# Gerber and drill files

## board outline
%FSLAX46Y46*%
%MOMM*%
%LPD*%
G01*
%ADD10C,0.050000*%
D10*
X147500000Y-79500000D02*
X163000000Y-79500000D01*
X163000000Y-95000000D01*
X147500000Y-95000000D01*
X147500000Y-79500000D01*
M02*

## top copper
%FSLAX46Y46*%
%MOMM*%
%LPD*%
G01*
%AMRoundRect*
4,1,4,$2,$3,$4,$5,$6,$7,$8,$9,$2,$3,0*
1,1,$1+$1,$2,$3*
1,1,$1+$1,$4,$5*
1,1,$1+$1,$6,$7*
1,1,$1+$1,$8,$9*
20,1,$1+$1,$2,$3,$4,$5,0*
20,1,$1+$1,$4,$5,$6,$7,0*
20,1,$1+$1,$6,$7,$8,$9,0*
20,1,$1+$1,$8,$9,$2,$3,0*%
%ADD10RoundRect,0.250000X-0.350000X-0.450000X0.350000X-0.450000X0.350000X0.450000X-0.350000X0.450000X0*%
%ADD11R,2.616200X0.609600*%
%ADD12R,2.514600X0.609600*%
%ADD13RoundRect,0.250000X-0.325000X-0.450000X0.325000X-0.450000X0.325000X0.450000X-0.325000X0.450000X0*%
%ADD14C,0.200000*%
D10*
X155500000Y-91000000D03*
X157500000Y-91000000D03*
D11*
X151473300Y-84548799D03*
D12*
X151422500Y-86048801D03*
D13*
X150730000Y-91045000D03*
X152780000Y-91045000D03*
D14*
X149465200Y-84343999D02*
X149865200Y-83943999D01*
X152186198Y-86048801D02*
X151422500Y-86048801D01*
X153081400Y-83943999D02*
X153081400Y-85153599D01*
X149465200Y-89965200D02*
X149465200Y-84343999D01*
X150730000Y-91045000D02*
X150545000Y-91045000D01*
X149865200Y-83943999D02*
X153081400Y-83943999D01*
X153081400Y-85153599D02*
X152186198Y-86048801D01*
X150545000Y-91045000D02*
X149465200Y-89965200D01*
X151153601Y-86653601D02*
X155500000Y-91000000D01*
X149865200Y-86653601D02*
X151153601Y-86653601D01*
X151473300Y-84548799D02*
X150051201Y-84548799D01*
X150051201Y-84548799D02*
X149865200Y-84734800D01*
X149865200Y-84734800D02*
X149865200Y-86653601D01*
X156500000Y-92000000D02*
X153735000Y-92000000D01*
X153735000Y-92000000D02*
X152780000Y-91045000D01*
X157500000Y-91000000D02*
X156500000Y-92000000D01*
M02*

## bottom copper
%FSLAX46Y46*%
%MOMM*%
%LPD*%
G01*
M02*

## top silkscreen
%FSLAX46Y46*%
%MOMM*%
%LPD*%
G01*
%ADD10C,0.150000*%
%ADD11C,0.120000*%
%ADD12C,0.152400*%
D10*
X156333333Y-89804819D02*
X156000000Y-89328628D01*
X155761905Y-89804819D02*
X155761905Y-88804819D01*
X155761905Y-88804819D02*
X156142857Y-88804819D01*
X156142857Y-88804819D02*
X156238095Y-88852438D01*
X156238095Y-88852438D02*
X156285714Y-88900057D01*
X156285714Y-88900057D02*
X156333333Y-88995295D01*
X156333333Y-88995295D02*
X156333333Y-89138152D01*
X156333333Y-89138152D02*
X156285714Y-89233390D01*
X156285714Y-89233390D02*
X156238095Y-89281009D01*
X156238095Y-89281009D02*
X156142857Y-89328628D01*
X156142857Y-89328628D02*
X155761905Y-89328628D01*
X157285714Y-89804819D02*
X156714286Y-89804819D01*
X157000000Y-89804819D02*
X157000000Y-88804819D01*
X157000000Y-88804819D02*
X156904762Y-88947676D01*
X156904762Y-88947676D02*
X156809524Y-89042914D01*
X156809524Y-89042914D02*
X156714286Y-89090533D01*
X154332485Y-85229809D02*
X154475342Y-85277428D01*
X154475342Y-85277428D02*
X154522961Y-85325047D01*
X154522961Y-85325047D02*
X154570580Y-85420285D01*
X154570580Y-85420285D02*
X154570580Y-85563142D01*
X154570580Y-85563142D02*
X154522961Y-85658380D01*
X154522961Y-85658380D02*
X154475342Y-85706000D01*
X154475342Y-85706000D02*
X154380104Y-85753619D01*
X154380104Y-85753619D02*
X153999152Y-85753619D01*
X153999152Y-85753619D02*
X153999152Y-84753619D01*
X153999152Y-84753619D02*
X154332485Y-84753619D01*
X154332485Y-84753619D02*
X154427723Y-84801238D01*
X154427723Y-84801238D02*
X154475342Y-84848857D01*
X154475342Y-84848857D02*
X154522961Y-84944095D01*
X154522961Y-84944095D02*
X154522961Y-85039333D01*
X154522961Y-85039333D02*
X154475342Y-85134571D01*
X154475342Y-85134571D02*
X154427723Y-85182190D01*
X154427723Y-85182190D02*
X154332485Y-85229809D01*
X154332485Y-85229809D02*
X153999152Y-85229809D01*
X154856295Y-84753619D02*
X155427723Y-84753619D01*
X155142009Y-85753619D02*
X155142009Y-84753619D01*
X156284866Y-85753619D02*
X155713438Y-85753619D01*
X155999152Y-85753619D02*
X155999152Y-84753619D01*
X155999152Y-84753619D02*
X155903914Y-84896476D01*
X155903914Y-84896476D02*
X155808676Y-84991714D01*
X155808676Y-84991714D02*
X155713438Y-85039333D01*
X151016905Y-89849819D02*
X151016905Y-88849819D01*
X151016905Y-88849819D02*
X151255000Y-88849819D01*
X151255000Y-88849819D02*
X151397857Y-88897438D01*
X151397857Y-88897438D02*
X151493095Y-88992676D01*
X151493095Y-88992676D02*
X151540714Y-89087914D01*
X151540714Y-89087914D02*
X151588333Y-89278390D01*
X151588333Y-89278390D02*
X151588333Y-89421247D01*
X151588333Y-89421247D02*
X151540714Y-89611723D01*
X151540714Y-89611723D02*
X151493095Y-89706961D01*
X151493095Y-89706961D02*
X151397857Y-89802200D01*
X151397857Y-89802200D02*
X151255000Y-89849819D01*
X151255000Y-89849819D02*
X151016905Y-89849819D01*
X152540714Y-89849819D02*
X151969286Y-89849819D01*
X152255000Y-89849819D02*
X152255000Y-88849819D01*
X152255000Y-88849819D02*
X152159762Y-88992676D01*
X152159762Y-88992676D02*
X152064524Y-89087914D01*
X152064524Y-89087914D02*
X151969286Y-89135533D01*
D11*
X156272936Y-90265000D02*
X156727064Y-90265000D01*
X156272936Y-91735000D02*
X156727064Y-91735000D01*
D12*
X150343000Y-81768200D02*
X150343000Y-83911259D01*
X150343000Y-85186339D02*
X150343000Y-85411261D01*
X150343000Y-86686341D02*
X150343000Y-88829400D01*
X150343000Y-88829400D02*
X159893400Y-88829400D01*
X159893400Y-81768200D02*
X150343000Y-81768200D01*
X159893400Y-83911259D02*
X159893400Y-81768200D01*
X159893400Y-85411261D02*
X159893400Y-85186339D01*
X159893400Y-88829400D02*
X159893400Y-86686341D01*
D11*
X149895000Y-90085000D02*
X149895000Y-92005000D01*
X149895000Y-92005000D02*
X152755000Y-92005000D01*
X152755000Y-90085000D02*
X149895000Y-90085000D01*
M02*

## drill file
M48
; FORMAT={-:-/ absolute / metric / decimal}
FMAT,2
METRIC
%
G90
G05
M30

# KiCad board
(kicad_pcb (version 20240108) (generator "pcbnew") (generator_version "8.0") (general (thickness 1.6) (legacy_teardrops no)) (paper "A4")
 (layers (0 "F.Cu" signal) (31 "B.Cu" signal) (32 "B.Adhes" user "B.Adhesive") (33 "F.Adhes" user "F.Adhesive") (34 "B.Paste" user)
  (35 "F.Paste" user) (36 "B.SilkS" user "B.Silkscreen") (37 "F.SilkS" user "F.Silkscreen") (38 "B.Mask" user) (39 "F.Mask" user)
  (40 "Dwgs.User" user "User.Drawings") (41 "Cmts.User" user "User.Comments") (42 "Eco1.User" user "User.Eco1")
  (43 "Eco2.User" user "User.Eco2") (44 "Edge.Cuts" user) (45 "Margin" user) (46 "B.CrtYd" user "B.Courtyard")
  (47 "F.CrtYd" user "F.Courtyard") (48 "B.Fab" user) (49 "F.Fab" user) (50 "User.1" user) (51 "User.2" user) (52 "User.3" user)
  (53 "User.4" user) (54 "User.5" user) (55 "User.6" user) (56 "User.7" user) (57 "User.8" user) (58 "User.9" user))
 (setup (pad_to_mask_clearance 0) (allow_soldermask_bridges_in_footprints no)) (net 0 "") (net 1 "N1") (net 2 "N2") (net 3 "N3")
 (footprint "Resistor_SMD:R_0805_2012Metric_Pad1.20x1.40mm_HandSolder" (layer "F.Cu") (at 156.5 91)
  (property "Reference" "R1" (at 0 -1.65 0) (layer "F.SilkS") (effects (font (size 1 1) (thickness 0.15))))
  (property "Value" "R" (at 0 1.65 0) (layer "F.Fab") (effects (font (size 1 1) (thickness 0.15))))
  (fp_line (start -0.227064 -0.735) (end 0.227064 -0.735) (stroke (width 0.12) (type solid)) (layer "F.SilkS"))
  (fp_line (start -0.227064 0.735) (end 0.227064 0.735) (stroke (width 0.12) (type solid)) (layer "F.SilkS"))
  (pad "1" smd roundrect (at -1 0) (size 1.2 1.4) (layers "F.Cu" "F.Paste" "F.Mask") (roundrect_rratio 0.208333) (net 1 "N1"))
  (pad "2" smd roundrect (at 1 0) (size 1.2 1.4) (layers "F.Cu" "F.Paste" "F.Mask") (roundrect_rratio 0.208333) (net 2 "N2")))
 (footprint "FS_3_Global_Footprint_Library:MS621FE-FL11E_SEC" (layer "F.Cu") (at 155.1182 85.2988)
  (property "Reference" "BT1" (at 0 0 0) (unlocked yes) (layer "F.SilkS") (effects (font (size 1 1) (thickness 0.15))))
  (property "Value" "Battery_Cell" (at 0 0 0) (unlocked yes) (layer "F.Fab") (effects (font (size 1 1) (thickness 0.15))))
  (fp_line (start -4.7752 -3.5306) (end -4.7752 -1.387541) (stroke (width 0.1524) (type solid)) (layer "F.SilkS"))
  (fp_line (start -4.7752 -0.112461) (end -4.7752 0.112461) (stroke (width 0.1524) (type solid)) (layer "F.SilkS"))
  (fp_line (start -4.7752 1.387541) (end -4.7752 3.5306) (stroke (width 0.1524) (type solid)) (layer "F.SilkS"))
  (fp_line (start -4.7752 3.5306) (end 4.7752 3.5306) (stroke (width 0.1524) (type solid)) (layer "F.SilkS"))
  (fp_line (start 4.7752 -3.5306) (end -4.7752 -3.5306) (stroke (width 0.1524) (type solid)) (layer "F.SilkS"))
  (fp_line (start 4.7752 -1.387541) (end 4.7752 -3.5306) (stroke (width 0.1524) (type solid)) (layer "F.SilkS"))
  (fp_line (start 4.7752 0.112461) (end 4.7752 -0.112461) (stroke (width 0.1524) (type solid)) (layer "F.SilkS"))
  (fp_line (start 4.7752 3.5306) (end 4.7752 1.387541) (stroke (width 0.1524) (type solid)) (layer "F.SilkS"))
  (pad "1" smd rect (at -3.6449 -0.750001) (size 2.6162 0.6096) (layers "F.Cu" "F.Paste" "F.Mask") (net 1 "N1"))
  (pad "2" smd rect (at -3.6957 0.750001) (size 2.5146 0.6096) (layers "F.Cu" "F.Paste" "F.Mask") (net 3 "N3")))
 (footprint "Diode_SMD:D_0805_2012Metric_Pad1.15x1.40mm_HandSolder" (layer "F.Cu") (at 151.755 91.045)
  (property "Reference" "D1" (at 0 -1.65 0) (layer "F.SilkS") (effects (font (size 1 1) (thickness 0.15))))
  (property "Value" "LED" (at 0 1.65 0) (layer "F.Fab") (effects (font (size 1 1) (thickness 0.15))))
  (fp_line (start -1.86 -0.96) (end -1.86 0.96) (stroke (width 0.12) (type solid)) (layer "F.SilkS"))
  (fp_line (start -1.86 0.96) (end 1 0.96) (stroke (width 0.12) (type solid)) (layer "F.SilkS"))
  (fp_line (start 1 -0.96) (end -1.86 -0.96) (stroke (width 0.12) (type solid)) (layer "F.SilkS"))
  (pad "1" smd roundrect (at -1.025 0) (size 1.15 1.4) (layers "F.Cu" "F.Paste" "F.Mask") (roundrect_rratio 0.217391) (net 3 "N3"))
  (pad "2" smd roundrect (at 1.025 0) (size 1.15 1.4) (layers "F.Cu" "F.Paste" "F.Mask") (roundrect_rratio 0.217391) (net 2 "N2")))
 (gr_rect (start 147.5 79.5) (end 163 95) (stroke (width 0.05) (type default)) (fill none) (layer "Edge.Cuts"))
 (segment (start 149.4652 84.343999) (end 149.8652 83.943999) (width 0.2) (layer "F.Cu") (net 3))
 (segment (start 152.186198 86.048801) (end 151.4225 86.048801) (width 0.2) (layer "F.Cu") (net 3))
 (segment (start 153.0814 83.943999) (end 153.0814 85.153599) (width 0.2) (layer "F.Cu") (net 3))
 (segment (start 149.4652 89.9652) (end 149.4652 84.343999) (width 0.2) (layer "F.Cu") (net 3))
 (segment (start 150.73 91.045) (end 150.545 91.045) (width 0.2) (layer "F.Cu") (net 3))
 (segment (start 149.8652 83.943999) (end 153.0814 83.943999) (width 0.2) (layer "F.Cu") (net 3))
 (segment (start 153.0814 85.153599) (end 152.186198 86.048801) (width 0.2) (layer "F.Cu") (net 3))
 (segment (start 150.545 91.045) (end 149.4652 89.9652) (width 0.2) (layer "F.Cu") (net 3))
 (segment (start 151.153601 86.653601) (end 155.5 91) (width 0.2) (layer "F.Cu") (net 1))
 (segment (start 149.8652 86.653601) (end 151.153601 86.653601) (width 0.2) (layer "F.Cu") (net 1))
 (segment (start 151.4733 84.548799) (end 150.051201 84.548799) (width 0.2) (layer "F.Cu") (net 1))
 (segment (start 150.051201 84.548799) (end 149.8652 84.7348) (width 0.2) (layer "F.Cu") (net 1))
 (segment (start 149.8652 84.7348) (end 149.8652 86.653601) (width 0.2) (layer "F.Cu") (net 1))
 (segment (start 156.5 92) (end 153.735 92) (width 0.2) (layer "F.Cu") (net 2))
 (segment (start 153.735 92) (end 152.78 91.045) (width 0.2) (layer "F.Cu") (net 2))
 (segment (start 157.5 91) (end 156.5 92) (width 0.2) (layer "F.Cu") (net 2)))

